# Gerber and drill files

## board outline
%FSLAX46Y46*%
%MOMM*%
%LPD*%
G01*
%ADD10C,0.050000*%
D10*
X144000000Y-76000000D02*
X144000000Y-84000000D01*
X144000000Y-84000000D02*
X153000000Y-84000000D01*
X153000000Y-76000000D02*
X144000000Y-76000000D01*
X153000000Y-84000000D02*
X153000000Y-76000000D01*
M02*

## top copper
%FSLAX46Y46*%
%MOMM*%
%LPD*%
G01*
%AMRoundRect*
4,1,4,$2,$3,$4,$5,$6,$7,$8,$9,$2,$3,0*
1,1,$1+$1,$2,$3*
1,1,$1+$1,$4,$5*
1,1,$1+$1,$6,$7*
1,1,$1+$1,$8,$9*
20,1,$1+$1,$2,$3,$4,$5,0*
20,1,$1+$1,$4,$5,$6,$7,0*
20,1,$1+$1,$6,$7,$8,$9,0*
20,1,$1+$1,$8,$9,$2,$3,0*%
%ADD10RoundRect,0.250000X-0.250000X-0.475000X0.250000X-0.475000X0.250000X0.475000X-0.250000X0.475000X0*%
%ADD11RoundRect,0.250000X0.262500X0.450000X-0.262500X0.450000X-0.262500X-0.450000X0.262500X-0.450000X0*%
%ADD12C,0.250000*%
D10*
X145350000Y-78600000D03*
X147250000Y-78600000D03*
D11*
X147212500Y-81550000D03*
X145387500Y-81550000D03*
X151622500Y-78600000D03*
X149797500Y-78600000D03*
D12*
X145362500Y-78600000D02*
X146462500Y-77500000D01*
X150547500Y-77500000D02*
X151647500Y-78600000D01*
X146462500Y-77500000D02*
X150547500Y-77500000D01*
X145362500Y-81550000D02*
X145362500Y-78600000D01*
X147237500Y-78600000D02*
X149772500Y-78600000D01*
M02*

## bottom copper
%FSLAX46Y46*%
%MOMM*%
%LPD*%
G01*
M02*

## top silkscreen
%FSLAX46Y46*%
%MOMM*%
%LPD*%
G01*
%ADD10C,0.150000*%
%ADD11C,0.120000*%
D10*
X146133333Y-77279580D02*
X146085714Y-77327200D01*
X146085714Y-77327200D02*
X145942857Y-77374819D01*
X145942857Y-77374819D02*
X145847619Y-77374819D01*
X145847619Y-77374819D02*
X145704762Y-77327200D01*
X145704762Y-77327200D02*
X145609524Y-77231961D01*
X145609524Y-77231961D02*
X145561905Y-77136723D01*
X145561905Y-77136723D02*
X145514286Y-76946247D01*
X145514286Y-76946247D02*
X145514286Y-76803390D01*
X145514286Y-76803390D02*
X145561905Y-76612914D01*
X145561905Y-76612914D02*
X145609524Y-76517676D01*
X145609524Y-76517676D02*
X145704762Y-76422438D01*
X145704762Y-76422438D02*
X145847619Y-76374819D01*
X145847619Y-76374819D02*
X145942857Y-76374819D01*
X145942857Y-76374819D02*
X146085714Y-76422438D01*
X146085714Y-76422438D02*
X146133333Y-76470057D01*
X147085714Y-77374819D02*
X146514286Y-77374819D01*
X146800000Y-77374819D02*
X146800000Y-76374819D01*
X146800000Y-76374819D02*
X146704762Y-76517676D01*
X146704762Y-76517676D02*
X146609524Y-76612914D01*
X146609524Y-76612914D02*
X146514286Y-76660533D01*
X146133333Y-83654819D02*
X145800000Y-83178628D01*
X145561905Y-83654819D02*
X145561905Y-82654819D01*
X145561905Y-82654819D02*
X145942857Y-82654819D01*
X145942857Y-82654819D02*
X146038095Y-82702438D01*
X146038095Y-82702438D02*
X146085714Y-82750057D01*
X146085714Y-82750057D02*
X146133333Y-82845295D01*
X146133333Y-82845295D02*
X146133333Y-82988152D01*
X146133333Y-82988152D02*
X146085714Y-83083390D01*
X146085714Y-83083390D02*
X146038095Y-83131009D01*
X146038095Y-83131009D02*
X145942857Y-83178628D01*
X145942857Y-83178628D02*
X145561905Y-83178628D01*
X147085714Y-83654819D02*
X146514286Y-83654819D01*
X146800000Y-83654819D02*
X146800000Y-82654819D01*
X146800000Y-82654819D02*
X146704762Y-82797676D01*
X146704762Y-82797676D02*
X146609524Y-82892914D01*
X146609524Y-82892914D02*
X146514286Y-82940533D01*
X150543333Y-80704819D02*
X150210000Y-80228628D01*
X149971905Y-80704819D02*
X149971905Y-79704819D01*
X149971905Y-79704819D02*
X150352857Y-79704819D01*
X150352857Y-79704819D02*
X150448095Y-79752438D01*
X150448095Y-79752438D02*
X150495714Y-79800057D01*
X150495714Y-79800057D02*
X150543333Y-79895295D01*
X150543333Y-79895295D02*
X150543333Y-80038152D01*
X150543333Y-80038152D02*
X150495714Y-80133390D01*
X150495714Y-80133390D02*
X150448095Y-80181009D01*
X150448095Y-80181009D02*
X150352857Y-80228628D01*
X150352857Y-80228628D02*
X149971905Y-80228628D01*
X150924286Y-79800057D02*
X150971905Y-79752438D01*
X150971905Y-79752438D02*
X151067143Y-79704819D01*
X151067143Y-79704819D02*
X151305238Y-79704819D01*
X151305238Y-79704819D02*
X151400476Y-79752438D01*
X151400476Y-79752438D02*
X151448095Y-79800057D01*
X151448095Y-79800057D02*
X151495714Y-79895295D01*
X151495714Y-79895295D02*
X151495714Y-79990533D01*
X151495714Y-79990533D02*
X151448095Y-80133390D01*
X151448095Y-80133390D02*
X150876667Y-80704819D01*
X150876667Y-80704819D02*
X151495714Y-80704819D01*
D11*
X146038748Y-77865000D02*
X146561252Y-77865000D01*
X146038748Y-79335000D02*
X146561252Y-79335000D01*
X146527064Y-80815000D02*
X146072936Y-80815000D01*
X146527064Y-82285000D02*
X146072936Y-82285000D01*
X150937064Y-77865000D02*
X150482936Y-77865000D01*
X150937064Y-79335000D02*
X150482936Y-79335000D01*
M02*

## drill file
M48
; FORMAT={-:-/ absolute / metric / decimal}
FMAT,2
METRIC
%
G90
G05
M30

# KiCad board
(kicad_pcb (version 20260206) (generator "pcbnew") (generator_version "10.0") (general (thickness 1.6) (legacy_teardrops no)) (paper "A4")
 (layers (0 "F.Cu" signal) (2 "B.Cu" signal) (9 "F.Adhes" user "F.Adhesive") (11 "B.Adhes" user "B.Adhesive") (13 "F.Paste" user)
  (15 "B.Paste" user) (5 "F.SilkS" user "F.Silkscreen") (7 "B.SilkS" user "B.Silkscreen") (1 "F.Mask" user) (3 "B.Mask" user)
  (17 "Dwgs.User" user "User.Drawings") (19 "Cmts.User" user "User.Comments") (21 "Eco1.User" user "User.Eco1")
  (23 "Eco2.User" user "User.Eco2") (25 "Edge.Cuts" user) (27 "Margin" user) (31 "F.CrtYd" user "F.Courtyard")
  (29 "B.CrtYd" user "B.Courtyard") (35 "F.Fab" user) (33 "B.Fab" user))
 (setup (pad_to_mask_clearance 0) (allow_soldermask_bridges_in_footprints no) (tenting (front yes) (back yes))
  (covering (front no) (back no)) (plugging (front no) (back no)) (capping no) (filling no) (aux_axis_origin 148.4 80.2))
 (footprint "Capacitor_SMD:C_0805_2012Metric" (layer "F.Cu") (at 146.3 78.6)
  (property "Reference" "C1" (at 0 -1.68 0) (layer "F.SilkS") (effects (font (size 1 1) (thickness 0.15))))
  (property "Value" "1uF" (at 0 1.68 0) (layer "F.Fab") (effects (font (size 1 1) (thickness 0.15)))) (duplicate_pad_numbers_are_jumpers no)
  (fp_line (start -0.261252 -0.735) (end 0.261252 -0.735) (stroke (width 0.12) (type solid)) (layer "F.SilkS"))
  (fp_line (start -0.261252 0.735) (end 0.261252 0.735) (stroke (width 0.12) (type solid)) (layer "F.SilkS"))
  (pad "1" smd roundrect (at -0.95 0) (size 1 1.45) (layers "F.Cu" "F.Mask" "F.Paste") (roundrect_rratio 0.25) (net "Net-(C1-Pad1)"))
  (pad "2" smd roundrect (at 0.95 0) (size 1 1.45) (layers "F.Cu" "F.Mask" "F.Paste") (roundrect_rratio 0.25) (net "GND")))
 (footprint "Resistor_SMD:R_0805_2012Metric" (layer "F.Cu") (at 146.3 81.55 180)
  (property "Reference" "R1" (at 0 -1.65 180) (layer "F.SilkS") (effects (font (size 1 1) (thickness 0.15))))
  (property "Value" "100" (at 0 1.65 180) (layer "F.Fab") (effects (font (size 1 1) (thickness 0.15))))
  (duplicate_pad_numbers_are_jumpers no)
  (fp_line (start -0.227064 0.735) (end 0.227064 0.735) (stroke (width 0.12) (type solid)) (layer "F.SilkS"))
  (fp_line (start -0.227064 -0.735) (end 0.227064 -0.735) (stroke (width 0.12) (type solid)) (layer "F.SilkS"))
  (pad "1" smd roundrect (at -0.9125 0 180) (size 1.025 1.4) (layers "F.Cu" "F.Mask" "F.Paste") (roundrect_rratio 0.243902) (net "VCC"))
  (pad "2" smd roundrect (at 0.9125 0 180) (size 1.025 1.4) (layers "F.Cu" "F.Mask" "F.Paste") (roundrect_rratio 0.243902)
   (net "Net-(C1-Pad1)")))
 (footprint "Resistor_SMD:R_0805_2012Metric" (layer "F.Cu") (at 150.71 78.6 180)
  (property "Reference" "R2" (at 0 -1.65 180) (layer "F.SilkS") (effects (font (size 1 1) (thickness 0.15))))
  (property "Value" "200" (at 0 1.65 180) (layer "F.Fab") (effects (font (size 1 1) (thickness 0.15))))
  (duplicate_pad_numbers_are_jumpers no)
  (fp_line (start -0.227064 0.735) (end 0.227064 0.735) (stroke (width 0.12) (type solid)) (layer "F.SilkS"))
  (fp_line (start -0.227064 -0.735) (end 0.227064 -0.735) (stroke (width 0.12) (type solid)) (layer "F.SilkS"))
  (pad "1" smd roundrect (at -0.9125 0 180) (size 1.025 1.4) (layers "F.Cu" "F.Mask" "F.Paste") (roundrect_rratio 0.243902)
   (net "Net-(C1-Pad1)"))
  (pad "2" smd roundrect (at 0.9125 0 180) (size 1.025 1.4) (layers "F.Cu" "F.Mask" "F.Paste") (roundrect_rratio 0.243902) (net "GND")))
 (gr_line (start 144 76) (end 144 84) (stroke (width 0.05) (type solid)) (layer "Edge.Cuts"))
 (gr_line (start 144 84) (end 153 84) (stroke (width 0.05) (type solid)) (layer "Edge.Cuts"))
 (gr_line (start 153 76) (end 144 76) (stroke (width 0.05) (type solid)) (layer "Edge.Cuts"))
 (gr_line (start 153 84) (end 153 76) (stroke (width 0.05) (type solid)) (layer "Edge.Cuts"))
 (segment (start 145.3625 78.6) (end 146.4625 77.5) (width 0.25) (layer "F.Cu") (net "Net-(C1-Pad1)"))
 (segment (start 150.5475 77.5) (end 151.6475 78.6) (width 0.25) (layer "F.Cu") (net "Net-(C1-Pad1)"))
 (segment (start 146.4625 77.5) (end 150.5475 77.5) (width 0.25) (layer "F.Cu") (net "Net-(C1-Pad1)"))
 (segment (start 145.3625 81.55) (end 145.3625 78.6) (width 0.25) (layer "F.Cu") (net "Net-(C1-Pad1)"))
 (segment (start 147.2375 78.6) (end 149.7725 78.6) (width 0.25) (layer "F.Cu") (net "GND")))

